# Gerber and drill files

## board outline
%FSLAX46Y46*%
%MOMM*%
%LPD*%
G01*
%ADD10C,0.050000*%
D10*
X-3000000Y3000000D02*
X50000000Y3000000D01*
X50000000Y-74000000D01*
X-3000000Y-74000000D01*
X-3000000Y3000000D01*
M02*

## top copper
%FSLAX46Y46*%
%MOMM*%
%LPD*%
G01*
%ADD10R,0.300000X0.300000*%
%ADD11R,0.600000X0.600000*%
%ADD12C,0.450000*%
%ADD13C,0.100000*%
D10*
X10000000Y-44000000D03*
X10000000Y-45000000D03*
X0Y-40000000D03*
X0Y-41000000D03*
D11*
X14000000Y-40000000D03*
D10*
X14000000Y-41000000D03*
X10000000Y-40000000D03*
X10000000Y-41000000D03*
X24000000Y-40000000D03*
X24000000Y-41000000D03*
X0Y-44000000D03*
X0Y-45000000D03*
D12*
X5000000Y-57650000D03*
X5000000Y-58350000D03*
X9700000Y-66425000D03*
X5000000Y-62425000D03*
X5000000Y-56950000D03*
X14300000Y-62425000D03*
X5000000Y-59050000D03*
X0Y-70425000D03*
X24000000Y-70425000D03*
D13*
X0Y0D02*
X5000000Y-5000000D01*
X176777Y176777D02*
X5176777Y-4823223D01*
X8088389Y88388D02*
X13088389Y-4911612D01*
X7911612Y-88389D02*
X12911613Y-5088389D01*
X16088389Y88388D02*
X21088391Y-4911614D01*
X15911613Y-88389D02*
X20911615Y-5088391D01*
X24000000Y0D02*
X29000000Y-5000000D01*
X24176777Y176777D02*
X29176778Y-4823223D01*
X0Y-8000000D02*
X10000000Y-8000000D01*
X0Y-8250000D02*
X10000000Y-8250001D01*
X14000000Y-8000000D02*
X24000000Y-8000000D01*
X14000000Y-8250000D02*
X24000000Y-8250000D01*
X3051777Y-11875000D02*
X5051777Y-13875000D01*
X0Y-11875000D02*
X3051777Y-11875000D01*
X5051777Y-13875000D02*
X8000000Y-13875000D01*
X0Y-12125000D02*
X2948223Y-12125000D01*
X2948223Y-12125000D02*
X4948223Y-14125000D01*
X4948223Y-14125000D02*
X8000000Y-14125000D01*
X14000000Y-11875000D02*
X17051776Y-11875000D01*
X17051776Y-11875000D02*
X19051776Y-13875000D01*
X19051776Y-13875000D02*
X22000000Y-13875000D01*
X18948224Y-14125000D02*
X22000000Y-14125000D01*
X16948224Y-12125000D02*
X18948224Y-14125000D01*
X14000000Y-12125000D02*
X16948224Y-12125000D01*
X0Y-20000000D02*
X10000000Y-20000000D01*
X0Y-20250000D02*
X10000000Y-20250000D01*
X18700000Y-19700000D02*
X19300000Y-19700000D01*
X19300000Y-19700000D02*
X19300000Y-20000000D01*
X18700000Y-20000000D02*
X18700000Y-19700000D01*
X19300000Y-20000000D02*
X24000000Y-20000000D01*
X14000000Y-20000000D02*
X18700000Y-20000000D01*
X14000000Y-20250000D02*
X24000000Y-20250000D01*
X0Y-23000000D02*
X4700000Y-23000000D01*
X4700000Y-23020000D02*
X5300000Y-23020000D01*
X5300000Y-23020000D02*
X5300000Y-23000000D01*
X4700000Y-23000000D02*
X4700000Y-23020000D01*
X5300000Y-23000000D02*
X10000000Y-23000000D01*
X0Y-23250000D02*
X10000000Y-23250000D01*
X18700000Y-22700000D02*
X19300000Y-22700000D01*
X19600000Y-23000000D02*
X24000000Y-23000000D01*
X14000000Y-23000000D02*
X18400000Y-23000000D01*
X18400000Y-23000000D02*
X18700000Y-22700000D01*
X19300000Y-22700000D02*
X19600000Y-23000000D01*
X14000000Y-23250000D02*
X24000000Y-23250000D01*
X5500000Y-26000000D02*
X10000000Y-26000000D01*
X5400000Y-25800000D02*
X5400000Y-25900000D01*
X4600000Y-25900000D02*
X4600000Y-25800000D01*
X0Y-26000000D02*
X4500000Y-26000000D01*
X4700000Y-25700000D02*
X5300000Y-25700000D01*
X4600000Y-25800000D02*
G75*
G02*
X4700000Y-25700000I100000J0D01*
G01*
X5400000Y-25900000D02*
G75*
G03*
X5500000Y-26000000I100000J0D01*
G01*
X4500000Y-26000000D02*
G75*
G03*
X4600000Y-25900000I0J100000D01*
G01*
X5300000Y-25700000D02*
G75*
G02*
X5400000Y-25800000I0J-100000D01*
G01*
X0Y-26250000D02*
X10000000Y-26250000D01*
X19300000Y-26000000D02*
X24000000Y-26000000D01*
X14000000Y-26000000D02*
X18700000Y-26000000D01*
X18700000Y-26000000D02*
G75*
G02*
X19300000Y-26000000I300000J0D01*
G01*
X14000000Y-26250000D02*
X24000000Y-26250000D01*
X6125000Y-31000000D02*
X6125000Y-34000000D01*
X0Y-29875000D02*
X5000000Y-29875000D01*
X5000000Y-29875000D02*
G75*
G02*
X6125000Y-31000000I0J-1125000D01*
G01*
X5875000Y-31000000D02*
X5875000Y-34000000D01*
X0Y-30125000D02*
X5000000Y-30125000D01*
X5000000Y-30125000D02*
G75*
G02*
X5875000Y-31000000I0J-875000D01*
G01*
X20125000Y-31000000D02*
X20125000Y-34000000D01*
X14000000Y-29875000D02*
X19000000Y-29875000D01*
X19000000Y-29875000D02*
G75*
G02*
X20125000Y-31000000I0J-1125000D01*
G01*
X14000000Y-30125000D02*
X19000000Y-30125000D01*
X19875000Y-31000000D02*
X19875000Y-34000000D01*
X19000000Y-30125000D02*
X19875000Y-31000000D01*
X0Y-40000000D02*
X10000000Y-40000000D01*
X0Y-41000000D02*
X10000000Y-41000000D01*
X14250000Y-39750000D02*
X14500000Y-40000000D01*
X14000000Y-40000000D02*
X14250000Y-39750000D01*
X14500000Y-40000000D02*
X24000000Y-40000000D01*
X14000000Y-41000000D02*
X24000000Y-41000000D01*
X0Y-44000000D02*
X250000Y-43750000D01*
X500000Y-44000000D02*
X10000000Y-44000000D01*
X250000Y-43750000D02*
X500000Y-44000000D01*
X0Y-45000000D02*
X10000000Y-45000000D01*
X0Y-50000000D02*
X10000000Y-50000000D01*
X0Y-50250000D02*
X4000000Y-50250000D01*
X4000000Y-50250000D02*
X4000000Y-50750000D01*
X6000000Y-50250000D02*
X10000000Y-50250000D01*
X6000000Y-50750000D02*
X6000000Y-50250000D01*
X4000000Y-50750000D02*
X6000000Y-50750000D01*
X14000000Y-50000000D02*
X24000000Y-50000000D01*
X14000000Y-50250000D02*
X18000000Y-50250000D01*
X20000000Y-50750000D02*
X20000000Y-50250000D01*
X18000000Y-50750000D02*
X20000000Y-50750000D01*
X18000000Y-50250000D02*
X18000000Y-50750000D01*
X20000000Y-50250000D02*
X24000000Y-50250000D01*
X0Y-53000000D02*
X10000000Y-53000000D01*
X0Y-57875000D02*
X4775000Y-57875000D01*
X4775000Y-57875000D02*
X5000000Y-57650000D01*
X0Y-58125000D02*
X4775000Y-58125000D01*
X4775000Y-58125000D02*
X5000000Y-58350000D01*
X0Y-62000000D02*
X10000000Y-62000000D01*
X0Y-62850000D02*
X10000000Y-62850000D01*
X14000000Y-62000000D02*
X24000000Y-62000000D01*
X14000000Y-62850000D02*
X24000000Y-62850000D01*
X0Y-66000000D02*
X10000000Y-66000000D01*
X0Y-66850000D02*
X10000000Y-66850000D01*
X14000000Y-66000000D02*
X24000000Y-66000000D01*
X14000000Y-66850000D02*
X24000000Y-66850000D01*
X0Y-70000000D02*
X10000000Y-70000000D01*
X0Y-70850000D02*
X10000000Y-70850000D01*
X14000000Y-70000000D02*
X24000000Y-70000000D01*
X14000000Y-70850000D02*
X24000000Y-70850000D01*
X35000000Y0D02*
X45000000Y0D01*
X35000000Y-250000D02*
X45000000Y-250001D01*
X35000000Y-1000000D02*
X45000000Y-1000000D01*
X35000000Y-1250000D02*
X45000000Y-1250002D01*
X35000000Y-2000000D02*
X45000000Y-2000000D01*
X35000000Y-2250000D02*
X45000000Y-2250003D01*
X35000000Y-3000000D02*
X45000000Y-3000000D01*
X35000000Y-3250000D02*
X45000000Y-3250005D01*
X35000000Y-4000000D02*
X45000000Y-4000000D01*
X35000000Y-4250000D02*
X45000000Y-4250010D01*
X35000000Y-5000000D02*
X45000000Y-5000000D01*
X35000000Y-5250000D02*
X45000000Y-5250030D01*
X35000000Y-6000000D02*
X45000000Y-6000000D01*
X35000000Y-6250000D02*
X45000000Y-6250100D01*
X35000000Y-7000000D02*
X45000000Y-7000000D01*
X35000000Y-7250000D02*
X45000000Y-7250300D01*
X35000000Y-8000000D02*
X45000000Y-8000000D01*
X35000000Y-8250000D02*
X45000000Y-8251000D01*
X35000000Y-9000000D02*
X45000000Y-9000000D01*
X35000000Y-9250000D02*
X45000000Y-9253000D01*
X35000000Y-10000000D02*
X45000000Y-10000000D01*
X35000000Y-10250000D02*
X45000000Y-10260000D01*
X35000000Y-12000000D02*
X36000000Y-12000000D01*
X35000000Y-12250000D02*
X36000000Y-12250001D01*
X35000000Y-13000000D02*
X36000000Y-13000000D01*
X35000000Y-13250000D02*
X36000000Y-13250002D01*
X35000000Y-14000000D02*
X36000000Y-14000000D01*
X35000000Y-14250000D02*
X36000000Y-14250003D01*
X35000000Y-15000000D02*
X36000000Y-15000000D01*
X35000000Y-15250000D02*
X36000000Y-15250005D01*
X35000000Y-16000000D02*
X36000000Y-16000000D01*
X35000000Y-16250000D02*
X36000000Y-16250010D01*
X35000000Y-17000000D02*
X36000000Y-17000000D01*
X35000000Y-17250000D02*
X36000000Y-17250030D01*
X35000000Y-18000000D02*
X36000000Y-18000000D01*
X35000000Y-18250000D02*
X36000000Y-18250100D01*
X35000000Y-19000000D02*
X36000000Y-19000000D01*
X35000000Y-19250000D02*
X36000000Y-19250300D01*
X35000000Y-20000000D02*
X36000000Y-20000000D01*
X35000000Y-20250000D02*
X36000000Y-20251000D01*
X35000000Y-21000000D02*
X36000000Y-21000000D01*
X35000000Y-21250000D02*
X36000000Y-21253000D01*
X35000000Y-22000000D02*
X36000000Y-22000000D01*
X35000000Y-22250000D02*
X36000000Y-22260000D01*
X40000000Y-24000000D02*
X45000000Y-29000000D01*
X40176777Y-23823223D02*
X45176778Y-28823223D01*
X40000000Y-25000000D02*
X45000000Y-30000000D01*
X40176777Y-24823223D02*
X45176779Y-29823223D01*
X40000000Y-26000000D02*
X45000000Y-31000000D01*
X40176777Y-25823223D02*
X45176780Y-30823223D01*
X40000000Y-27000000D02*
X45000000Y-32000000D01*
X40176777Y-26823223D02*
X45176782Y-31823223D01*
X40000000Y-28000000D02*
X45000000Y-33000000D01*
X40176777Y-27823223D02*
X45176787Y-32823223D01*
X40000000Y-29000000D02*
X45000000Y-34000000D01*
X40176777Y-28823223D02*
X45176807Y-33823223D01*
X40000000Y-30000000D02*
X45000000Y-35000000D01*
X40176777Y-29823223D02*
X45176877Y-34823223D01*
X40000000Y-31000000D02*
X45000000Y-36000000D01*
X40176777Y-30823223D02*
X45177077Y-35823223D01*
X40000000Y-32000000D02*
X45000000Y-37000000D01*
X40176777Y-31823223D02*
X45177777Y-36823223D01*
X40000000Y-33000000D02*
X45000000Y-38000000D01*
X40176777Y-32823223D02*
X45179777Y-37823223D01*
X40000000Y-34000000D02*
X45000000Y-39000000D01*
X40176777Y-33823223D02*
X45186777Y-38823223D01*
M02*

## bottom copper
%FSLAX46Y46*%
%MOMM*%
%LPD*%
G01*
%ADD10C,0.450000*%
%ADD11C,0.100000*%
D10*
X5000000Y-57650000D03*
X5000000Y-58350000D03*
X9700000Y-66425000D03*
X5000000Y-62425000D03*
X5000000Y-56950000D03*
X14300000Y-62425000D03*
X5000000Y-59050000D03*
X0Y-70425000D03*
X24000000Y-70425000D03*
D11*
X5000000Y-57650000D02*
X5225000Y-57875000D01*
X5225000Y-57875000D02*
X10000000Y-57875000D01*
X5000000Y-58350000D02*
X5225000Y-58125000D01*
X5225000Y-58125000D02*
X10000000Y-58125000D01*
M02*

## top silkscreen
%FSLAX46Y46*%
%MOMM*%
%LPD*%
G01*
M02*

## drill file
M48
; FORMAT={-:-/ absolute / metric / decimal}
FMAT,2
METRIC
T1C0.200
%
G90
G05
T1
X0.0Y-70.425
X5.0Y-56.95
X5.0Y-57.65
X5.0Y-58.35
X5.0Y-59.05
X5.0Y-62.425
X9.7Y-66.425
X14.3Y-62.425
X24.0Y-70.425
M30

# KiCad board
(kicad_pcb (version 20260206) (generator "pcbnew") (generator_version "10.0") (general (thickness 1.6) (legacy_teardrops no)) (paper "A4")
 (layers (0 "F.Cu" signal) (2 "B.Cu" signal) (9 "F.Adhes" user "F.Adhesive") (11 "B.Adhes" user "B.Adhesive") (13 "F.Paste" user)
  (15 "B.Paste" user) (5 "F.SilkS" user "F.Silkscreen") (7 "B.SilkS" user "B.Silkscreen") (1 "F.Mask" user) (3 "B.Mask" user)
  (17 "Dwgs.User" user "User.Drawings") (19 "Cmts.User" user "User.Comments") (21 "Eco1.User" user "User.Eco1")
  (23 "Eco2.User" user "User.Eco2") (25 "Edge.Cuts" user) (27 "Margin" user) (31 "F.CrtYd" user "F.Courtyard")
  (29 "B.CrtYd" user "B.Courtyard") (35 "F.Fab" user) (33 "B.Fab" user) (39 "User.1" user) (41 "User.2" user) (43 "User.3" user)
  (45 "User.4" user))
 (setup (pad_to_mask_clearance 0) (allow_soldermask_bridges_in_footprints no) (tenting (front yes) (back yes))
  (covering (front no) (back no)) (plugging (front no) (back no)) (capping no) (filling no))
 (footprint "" (layer "F.Cu") (at 10 44)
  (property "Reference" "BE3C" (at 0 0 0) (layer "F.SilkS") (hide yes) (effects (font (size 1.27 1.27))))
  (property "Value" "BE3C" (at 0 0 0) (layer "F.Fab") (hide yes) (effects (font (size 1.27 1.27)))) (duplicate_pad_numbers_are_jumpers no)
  (pad "1" smd rect (at 0 0) (size 0.3 0.3) (layers "F.Cu" "F.Mask" "F.Paste") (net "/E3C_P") (thermal_bridge_angle 45))
  (pad "2" smd rect (at 0 1) (size 0.3 0.3) (layers "F.Cu" "F.Mask" "F.Paste") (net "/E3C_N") (thermal_bridge_angle 45)))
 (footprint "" (layer "F.Cu") (at 0 40)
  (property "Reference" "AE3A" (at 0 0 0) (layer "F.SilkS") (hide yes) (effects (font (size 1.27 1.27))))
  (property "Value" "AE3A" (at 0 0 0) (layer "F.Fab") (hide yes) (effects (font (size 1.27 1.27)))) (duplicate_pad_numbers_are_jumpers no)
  (pad "1" smd rect (at 0 0) (size 0.3 0.3) (layers "F.Cu" "F.Mask" "F.Paste") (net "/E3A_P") (die_length 1) (thermal_bridge_angle 45))
  (pad "2" smd rect (at 0 1) (size 0.3 0.3) (layers "F.Cu" "F.Mask" "F.Paste") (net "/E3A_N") (thermal_bridge_angle 45)))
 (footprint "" (layer "F.Cu") (at 14 40)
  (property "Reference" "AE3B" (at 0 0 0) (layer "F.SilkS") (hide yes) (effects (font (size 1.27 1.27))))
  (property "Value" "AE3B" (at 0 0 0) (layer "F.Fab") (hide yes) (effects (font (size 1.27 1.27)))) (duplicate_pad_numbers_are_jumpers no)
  (pad "1" smd rect (at 0 0) (size 0.6 0.6) (layers "F.Cu" "F.Mask" "F.Paste") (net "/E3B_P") (thermal_bridge_angle 45))
  (pad "2" smd rect (at 0 1) (size 0.3 0.3) (layers "F.Cu" "F.Mask" "F.Paste") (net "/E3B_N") (thermal_bridge_angle 45)))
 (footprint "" (layer "F.Cu") (at 10 40)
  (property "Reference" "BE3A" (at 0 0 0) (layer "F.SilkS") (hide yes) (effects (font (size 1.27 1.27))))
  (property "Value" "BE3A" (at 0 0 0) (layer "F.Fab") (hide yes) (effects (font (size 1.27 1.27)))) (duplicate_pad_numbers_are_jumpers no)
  (pad "1" smd rect (at 0 0) (size 0.3 0.3) (layers "F.Cu" "F.Mask" "F.Paste") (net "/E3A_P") (thermal_bridge_angle 45))
  (pad "2" smd rect (at 0 1) (size 0.3 0.3) (layers "F.Cu" "F.Mask" "F.Paste") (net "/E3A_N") (thermal_bridge_angle 45)))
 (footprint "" (layer "F.Cu") (at 24 40)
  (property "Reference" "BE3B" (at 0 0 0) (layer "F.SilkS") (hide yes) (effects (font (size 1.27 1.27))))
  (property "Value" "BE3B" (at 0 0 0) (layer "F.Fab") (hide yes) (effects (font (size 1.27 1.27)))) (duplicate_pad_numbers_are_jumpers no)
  (pad "1" smd rect (at 0 0) (size 0.3 0.3) (layers "F.Cu" "F.Mask" "F.Paste") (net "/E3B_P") (thermal_bridge_angle 45))
  (pad "2" smd rect (at 0 1) (size 0.3 0.3) (layers "F.Cu" "F.Mask" "F.Paste") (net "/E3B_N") (thermal_bridge_angle 45)))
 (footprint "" (layer "F.Cu") (at 0 44)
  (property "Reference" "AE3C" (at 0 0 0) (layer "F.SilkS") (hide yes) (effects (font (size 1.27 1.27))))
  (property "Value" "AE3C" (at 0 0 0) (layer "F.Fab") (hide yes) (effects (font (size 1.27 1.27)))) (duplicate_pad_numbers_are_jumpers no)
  (pad "1" smd rect (at 0 0) (size 0.3 0.3) (layers "F.Cu" "F.Mask" "F.Paste") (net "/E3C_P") (thermal_bridge_angle 45))
  (pad "2" smd rect (at 0 1) (size 0.3 0.3) (layers "F.Cu" "F.Mask" "F.Paste") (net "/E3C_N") (thermal_bridge_angle 45)))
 (gr_rect (start -3 -3) (end 50 74) (stroke (width 0.05) (type default)) (fill no) (layer "Edge.Cuts"))
 (segment (start 0 0) (end 5 5) (width 0.1) (layer "F.Cu") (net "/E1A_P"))
 (segment (start 0.176777 -0.176777) (end 5.176777 4.823223) (width 0.1) (layer "F.Cu") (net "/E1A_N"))
 (segment (start 8.088389 -0.088388) (end 13.088389 4.911612) (width 0.1) (layer "F.Cu") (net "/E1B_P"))
 (segment (start 7.911612 0.088389) (end 12.911613 5.088389) (width 0.1) (layer "F.Cu") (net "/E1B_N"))
 (segment (start 16.088389 -0.088388) (end 21.088391 4.911614) (width 0.1) (layer "F.Cu") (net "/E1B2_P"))
 (segment (start 15.911613 0.088389) (end 20.911615 5.088391) (width 0.1) (layer "F.Cu") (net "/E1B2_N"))
 (segment (start 24 0) (end 29 5) (width 0.1) (layer "F.Cu") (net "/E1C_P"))
 (segment (start 24.176777 -0.176777) (end 29.176778 4.823223) (width 0.1) (layer "F.Cu") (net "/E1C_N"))
 (segment (start 0 8) (end 10 8) (width 0.1) (layer "F.Cu") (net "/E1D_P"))
 (segment (start 0 8.25) (end 10 8.250001) (width 0.1) (layer "F.Cu") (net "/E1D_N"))
 (segment (start 14 8) (end 24 8) (width 0.1) (layer "F.Cu") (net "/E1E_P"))
 (segment (start 14 8.25) (end 24 8.25) (width 0.1) (layer "F.Cu") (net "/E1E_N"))
 (segment (start 3.051777 11.875) (end 5.051777 13.875) (width 0.1) (layer "F.Cu") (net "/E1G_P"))
 (segment (start 0 11.875) (end 3.051777 11.875) (width 0.1) (layer "F.Cu") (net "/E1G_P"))
 (segment (start 5.051777 13.875) (end 8 13.875) (width 0.1) (layer "F.Cu") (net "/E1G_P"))
 (segment (start 0 12.125) (end 2.948223 12.125) (width 0.1) (layer "F.Cu") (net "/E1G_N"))
 (segment (start 2.948223 12.125) (end 4.948223 14.125) (width 0.1) (layer "F.Cu") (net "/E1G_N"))
 (segment (start 4.948223 14.125) (end 8 14.125) (width 0.1) (layer "F.Cu") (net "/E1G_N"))
 (segment (start 14 11.875) (end 17.051776 11.875) (width 0.1) (layer "F.Cu") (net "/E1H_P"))
 (segment (start 17.051776 11.875) (end 19.051776 13.875) (width 0.1) (layer "F.Cu") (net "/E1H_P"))
 (segment (start 19.051776 13.875) (end 22 13.875) (width 0.1) (layer "F.Cu") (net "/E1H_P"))
 (segment (start 18.948224 14.125) (end 22 14.125) (width 0.1) (layer "F.Cu") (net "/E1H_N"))
 (segment (start 16.948224 12.125) (end 18.948224 14.125) (width 0.1) (layer "F.Cu") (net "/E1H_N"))
 (segment (start 14 12.125) (end 16.948224 12.125) (width 0.1) (layer "F.Cu") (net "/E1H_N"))
 (segment (start 0 20) (end 10 20) (width 0.1) (layer "F.Cu") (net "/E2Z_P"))
 (segment (start 0 20.25) (end 10 20.25) (width 0.1) (layer "F.Cu") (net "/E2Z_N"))
 (segment (start 18.7 19.7) (end 19.3 19.7) (width 0.1) (layer "F.Cu") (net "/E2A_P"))
 (segment (start 19.3 19.7) (end 19.3 20) (width 0.1) (layer "F.Cu") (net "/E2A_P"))
 (segment (start 18.7 20) (end 18.7 19.7) (width 0.1) (layer "F.Cu") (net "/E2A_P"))
 (segment (start 19.3 20) (end 24 20) (width 0.1) (layer "F.Cu") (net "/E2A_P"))
 (segment (start 14 20) (end 18.7 20) (width 0.1) (layer "F.Cu") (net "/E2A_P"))
 (segment (start 14 20.25) (end 24 20.25) (width 0.1) (layer "F.Cu") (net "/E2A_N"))
 (segment (start 0 23) (end 4.7 23) (width 0.1) (layer "F.Cu") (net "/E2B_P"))
 (segment (start 4.7 23.02) (end 5.3 23.02) (width 0.1) (layer "F.Cu") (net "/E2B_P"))
 (segment (start 5.3 23.02) (end 5.3 23) (width 0.1) (layer "F.Cu") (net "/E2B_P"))
 (segment (start 4.7 23) (end 4.7 23.02) (width 0.1) (layer "F.Cu") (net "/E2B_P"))
 (segment (start 5.3 23) (end 10 23) (width 0.1) (layer "F.Cu") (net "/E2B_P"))
 (segment (start 0 23.25) (end 10 23.25) (width 0.1) (layer "F.Cu") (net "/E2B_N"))
 (segment (start 18.7 22.7) (end 19.3 22.7) (width 0.1) (layer "F.Cu") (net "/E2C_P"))
 (segment (start 19.6 23) (end 24 23) (width 0.1) (layer "F.Cu") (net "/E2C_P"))
 (segment (start 14 23) (end 18.4 23) (width 0.1) (layer "F.Cu") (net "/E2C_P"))
 (segment (start 18.4 23) (end 18.7 22.7) (width 0.1) (layer "F.Cu") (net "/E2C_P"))
 (segment (start 19.3 22.7) (end 19.6 23) (width 0.1) (layer "F.Cu") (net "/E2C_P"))
 (segment (start 14 23.25) (end 24 23.25) (width 0.1) (layer "F.Cu") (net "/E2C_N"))
 (segment (start 5.5 26) (end 10 26) (width 0.1) (layer "F.Cu") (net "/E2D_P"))
 (segment (start 5.4 25.8) (end 5.4 25.9) (width 0.1) (layer "F.Cu") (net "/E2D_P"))
 (segment (start 4.6 25.9) (end 4.6 25.8) (width 0.1) (layer "F.Cu") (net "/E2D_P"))
 (segment (start 0 26) (end 4.5 26) (width 0.1) (layer "F.Cu") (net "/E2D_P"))
 (segment (start 4.7 25.7) (end 5.3 25.7) (width 0.1) (layer "F.Cu") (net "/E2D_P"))
 (arc (start 4.6 25.8) (mid 4.629289 25.729289) (end 4.7 25.7) (width 0.1) (layer "F.Cu") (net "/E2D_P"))
 (arc (start 5.4 25.9) (mid 5.429289 25.970711) (end 5.5 26) (width 0.1) (layer "F.Cu") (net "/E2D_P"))
 (arc (start 4.5 26) (mid 4.570711 25.970711) (end 4.6 25.9) (width 0.1) (layer "F.Cu") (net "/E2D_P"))
 (arc (start 5.3 25.7) (mid 5.370711 25.729289) (end 5.4 25.8) (width 0.1) (layer "F.Cu") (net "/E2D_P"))
 (segment (start 0 26.25) (end 10 26.25) (width 0.1) (layer "F.Cu") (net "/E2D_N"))
 (segment (start 19.3 26) (end 24 26) (width 0.1) (layer "F.Cu") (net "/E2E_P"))
 (segment (start 14 26) (end 18.7 26) (width 0.1) (layer "F.Cu") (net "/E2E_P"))
 (arc (start 18.7 26) (mid 19 25.7) (end 19.3 26) (width 0.1) (layer "F.Cu") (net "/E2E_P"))
 (segment (start 14 26.25) (end 24 26.25) (width 0.1) (layer "F.Cu") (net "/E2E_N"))
 (segment (start 6.125 31) (end 6.125 34) (width 0.1) (layer "F.Cu") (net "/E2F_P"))
 (segment (start 0 29.875) (end 5 29.875) (width 0.1) (layer "F.Cu") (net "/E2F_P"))
 (arc (start 5 29.875) (mid 5.795495 30.204505) (end 6.125 31) (width 0.1) (layer "F.Cu") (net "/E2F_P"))
 (segment (start 5.875 31) (end 5.875 34) (width 0.1) (layer "F.Cu") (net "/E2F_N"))
 (segment (start 0 30.125) (end 5 30.125) (width 0.1) (layer "F.Cu") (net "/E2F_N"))
 (arc (start 5 30.125) (mid 5.618718 30.381282) (end 5.875 31) (width 0.1) (layer "F.Cu") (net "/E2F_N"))
 (segment (start 20.125 31) (end 20.125 34) (width 0.1) (layer "F.Cu") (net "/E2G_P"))
 (segment (start 14 29.875) (end 19 29.875) (width 0.1) (layer "F.Cu") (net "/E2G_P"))
 (arc (start 19 29.875) (mid 19.795495 30.204505) (end 20.125 31) (width 0.1) (layer "F.Cu") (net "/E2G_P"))
 (segment (start 14 30.125) (end 19 30.125) (width 0.1) (layer "F.Cu") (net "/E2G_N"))
 (segment (start 19.875 31) (end 19.875 34) (width 0.1) (layer "F.Cu") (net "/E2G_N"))
 (segment (start 19 30.125) (end 19.875 31) (width 0.1) (layer "F.Cu") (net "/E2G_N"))
 (segment (start 0 40) (end 10 40) (width 0.1) (layer "F.Cu") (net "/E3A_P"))
 (segment (start 0 41) (end 10 41) (width 0.1) (layer "F.Cu") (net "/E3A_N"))
 (segment (start 14.25 39.75) (end 14.5 40) (width 0.1) (layer "F.Cu") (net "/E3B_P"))
 (segment (start 14 40) (end 14.25 39.75) (width 0.1) (layer "F.Cu") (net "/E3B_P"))
 (segment (start 14.5 40) (end 24 40) (width 0.1) (layer "F.Cu") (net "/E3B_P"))
 (segment (start 14 41) (end 24 41) (width 0.1) (layer "F.Cu") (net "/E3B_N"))
 (segment (start 0 44) (end 0.25 43.75) (width 0.1) (layer "F.Cu") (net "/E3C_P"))
 (segment (start 0.5 44) (end 10 44) (width 0.1) (layer "F.Cu") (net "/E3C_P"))
 (segment (start 0.25 43.75) (end 0.5 44) (width 0.1) (layer "F.Cu") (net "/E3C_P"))
 (segment (start 0 45) (end 10 45) (width 0.1) (layer "F.Cu") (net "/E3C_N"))
 (segment (start 0 50) (end 10 50) (width 0.1) (layer "F.Cu") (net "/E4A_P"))
 (segment (start 0 50.25) (end 4 50.25) (width 0.1) (layer "F.Cu") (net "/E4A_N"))
 (segment (start 4 50.25) (end 4 50.75) (width 0.1) (layer "F.Cu") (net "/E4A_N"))
 (segment (start 6 50.25) (end 10 50.25) (width 0.1) (layer "F.Cu") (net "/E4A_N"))
 (segment (start 6 50.75) (end 6 50.25) (width 0.1) (layer "F.Cu") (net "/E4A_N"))
 (segment (start 4 50.75) (end 6 50.75) (width 0.1) (layer "F.Cu") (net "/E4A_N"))
 (segment (start 14 50) (end 24 50) (width 0.1) (layer "F.Cu") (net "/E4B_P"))
 (segment (start 14 50.25) (end 18 50.25) (width 0.1) (layer "F.Cu") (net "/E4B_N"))
 (segment (start 20 50.75) (end 20 50.25) (width 0.1) (layer "F.Cu") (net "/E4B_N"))
 (segment (start 18 50.75) (end 20 50.75) (width 0.1) (layer "F.Cu") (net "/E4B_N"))
 (segment (start 18 50.25) (end 18 50.75) (width 0.1) (layer "F.Cu") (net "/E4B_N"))
 (segment (start 20 50.25) (end 24 50.25) (width 0.1) (layer "F.Cu") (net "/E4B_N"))
 (segment (start 0 53) (end 10 53) (width 0.1) (layer "F.Cu") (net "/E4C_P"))
 (segment (start 0 57.875) (end 4.775 57.875) (width 0.1) (layer "F.Cu") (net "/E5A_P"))
 (segment (start 4.775 57.875) (end 5 57.65) (width 0.1) (layer "F.Cu") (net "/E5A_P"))
 (via (at 5 57.65) (size 0.45) (drill 0.2) (layers "F.Cu" "B.Cu") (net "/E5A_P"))
 (segment (start 5 57.65) (end 5.225 57.875) (width 0.1) (layer "B.Cu") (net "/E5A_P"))
 (segment (start 5.225 57.875) (end 10 57.875) (width 0.1) (layer "B.Cu") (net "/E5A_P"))
 (segment (start 0 58.125) (end 4.775 58.125) (width 0.1) (layer "F.Cu") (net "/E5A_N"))
 (segment (start 4.775 58.125) (end 5 58.35) (width 0.1) (layer "F.Cu") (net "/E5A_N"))
 (via (at 5 58.35) (size 0.45) (drill 0.2) (layers "F.Cu" "B.Cu") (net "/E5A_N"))
 (segment (start 5 58.35) (end 5.225 58.125) (width 0.1) (layer "B.Cu") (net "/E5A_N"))
 (segment (start 5.225 58.125) (end 10 58.125) (width 0.1) (layer "B.Cu") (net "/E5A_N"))
 (via (at 9.7 66.425) (size 0.45) (drill 0.2) (layers "F.Cu" "B.Cu") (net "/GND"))
 (via (at 5 62.425) (size 0.45) (drill 0.2) (layers "F.Cu" "B.Cu") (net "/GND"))
 (via (at 5 56.95) (size 0.45) (drill 0.2) (layers "F.Cu" "B.Cu") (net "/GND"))
 (via (at 14.3 62.425) (size 0.45) (drill 0.2) (layers "F.Cu" "B.Cu") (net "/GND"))
 (via (at 5 59.05) (size 0.45) (drill 0.2) (layers "F.Cu" "B.Cu") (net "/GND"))
 (via (at 0 70.425) (size 0.45) (drill 0.2) (layers "F.Cu" "B.Cu") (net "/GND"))
 (via (at 24 70.425) (size 0.45) (drill 0.2) (layers "F.Cu" "B.Cu") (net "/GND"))
 (segment (start 0 62) (end 10 62) (width 0.1) (layer "F.Cu") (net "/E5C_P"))
 (segment (start 0 62.85) (end 10 62.85) (width 0.1) (layer "F.Cu") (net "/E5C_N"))
 (segment (start 14 62) (end 24 62) (width 0.1) (layer "F.Cu") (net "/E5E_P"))
 (segment (start 14 62.85) (end 24 62.85) (width 0.1) (layer "F.Cu") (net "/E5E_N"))
 (segment (start 0 66) (end 10 66) (width 0.1) (layer "F.Cu") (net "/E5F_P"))
 (segment (start 0 66.85) (end 10 66.85) (width 0.1) (layer "F.Cu") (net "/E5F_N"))
 (segment (start 14 66) (end 24 66) (width 0.1) (layer "F.Cu") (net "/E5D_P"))
 (segment (start 14 66.85) (end 24 66.85) (width 0.1) (layer "F.Cu") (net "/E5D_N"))
 (segment (start 0 70) (end 10 70) (width 0.1) (layer "F.Cu") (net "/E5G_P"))
 (segment (start 0 70.85) (end 10 70.85) (width 0.1) (layer "F.Cu") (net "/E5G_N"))
 (segment (start 14 70) (end 24 70) (width 0.1) (layer "F.Cu") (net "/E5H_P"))
 (segment (start 14 70.85) (end 24 70.85) (width 0.1) (layer "F.Cu") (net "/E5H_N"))
 (segment (start 35 0) (end 45 0) (width 0.1) (layer "F.Cu") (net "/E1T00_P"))
 (segment (start 35 0.25) (end 45 0.250001) (width 0.1) (layer "F.Cu") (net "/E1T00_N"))
 (segment (start 35 1) (end 45 1) (width 0.1) (layer "F.Cu") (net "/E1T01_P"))
 (segment (start 35 1.25) (end 45 1.250002) (width 0.1) (layer "F.Cu") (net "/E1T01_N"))
 (segment (start 35 2) (end 45 2) (width 0.1) (layer "F.Cu") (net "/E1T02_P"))
 (segment (start 35 2.25) (end 45 2.250003) (width 0.1) (layer "F.Cu") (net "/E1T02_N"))
 (segment (start 35 3) (end 45 3) (width 0.1) (layer "F.Cu") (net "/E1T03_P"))
 (segment (start 35 3.25) (end 45 3.250005) (width 0.1) (layer "F.Cu") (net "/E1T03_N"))
 (segment (start 35 4) (end 45 4) (width 0.1) (layer "F.Cu") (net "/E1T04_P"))
 (segment (start 35 4.25) (end 45 4.25001) (width 0.1) (layer "F.Cu") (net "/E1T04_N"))
 (segment (start 35 5) (end 45 5) (width 0.1) (layer "F.Cu") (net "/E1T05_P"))
 (segment (start 35 5.25) (end 45 5.25003) (width 0.1) (layer "F.Cu") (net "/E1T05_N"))
 (segment (start 35 6) (end 45 6) (width 0.1) (layer "F.Cu") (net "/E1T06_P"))
 (segment (start 35 6.25) (end 45 6.2501) (width 0.1) (layer "F.Cu") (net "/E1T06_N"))
 (segment (start 35 7) (end 45 7) (width 0.1) (layer "F.Cu") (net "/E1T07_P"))
 (segment (start 35 7.25) (end 45 7.2503) (width 0.1) (layer "F.Cu") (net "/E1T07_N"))
 (segment (start 35 8) (end 45 8) (width 0.1) (layer "F.Cu") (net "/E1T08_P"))
 (segment (start 35 8.25) (end 45 8.251) (width 0.1) (layer "F.Cu") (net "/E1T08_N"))
 (segment (start 35 9) (end 45 9) (width 0.1) (layer "F.Cu") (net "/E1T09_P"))
 (segment (start 35 9.25) (end 45 9.253) (width 0.1) (layer "F.Cu") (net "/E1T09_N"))
 (segment (start 35 10) (end 45 10) (width 0.1) (layer "F.Cu") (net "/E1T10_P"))
 (segment (start 35 10.25) (end 45 10.26) (width 0.1) (layer "F.Cu") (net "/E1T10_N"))
 (segment (start 35 12) (end 36 12) (width 0.1) (layer "F.Cu") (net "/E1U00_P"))
 (segment (start 35 12.25) (end 36 12.250001) (width 0.1) (layer "F.Cu") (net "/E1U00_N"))
 (segment (start 35 13) (end 36 13) (width 0.1) (layer "F.Cu") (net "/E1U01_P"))
 (segment (start 35 13.25) (end 36 13.250002) (width 0.1) (layer "F.Cu") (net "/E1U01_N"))
 (segment (start 35 14) (end 36 14) (width 0.1) (layer "F.Cu") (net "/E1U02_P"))
 (segment (start 35 14.25) (end 36 14.250003) (width 0.1) (layer "F.Cu") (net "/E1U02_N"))
 (segment (start 35 15) (end 36 15) (width 0.1) (layer "F.Cu") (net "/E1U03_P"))
 (segment (start 35 15.25) (end 36 15.250005) (width 0.1) (layer "F.Cu") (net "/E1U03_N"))
 (segment (start 35 16) (end 36 16) (width 0.1) (layer "F.Cu") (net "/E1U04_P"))
 (segment (start 35 16.25) (end 36 16.25001) (width 0.1) (layer "F.Cu") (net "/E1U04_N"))
 (segment (start 35 17) (end 36 17) (width 0.1) (layer "F.Cu") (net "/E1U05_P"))
 (segment (start 35 17.25) (end 36 17.25003) (width 0.1) (layer "F.Cu") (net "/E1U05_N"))
 (segment (start 35 18) (end 36 18) (width 0.1) (layer "F.Cu") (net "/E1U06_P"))
 (segment (start 35 18.25) (end 36 18.2501) (width 0.1) (layer "F.Cu") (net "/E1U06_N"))
 (segment (start 35 19) (end 36 19) (width 0.1) (layer "F.Cu") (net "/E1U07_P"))
 (segment (start 35 19.25) (end 36 19.2503) (width 0.1) (layer "F.Cu") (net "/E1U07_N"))
 (segment (start 35 20) (end 36 20) (width 0.1) (layer "F.Cu") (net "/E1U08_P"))
 (segment (start 35 20.25) (end 36 20.251) (width 0.1) (layer "F.Cu") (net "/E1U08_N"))
 (segment (start 35 21) (end 36 21) (width 0.1) (layer "F.Cu") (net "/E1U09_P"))
 (segment (start 35 21.25) (end 36 21.253) (width 0.1) (layer "F.Cu") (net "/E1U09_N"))
 (segment (start 35 22) (end 36 22) (width 0.1) (layer "F.Cu") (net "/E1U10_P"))
 (segment (start 35 22.25) (end 36 22.26) (width 0.1) (layer "F.Cu") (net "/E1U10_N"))
 (segment (start 40 24) (end 45 29) (width 0.1) (layer "F.Cu") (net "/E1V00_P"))
 (segment (start 40.176777 23.823223) (end 45.176778 28.823223) (width 0.1) (layer "F.Cu") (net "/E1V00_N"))
 (segment (start 40 25) (end 45 30) (width 0.1) (layer "F.Cu") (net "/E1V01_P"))
 (segment (start 40.176777 24.823223) (end 45.176779 29.823223) (width 0.1) (layer "F.Cu") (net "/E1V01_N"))
 (segment (start 40 26) (end 45 31) (width 0.1) (layer "F.Cu") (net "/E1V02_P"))
 (segment (start 40.176777 25.823223) (end 45.17678 30.823223) (width 0.1) (layer "F.Cu") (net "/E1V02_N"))
 (segment (start 40 27) (end 45 32) (width 0.1) (layer "F.Cu") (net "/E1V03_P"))
 (segment (start 40.176777 26.823223) (end 45.176782 31.823223) (width 0.1) (layer "F.Cu") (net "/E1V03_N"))
 (segment (start 40 28) (end 45 33) (width 0.1) (layer "F.Cu") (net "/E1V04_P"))
 (segment (start 40.176777 27.823223) (end 45.176787 32.823223) (width 0.1) (layer "F.Cu") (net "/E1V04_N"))
 (segment (start 40 29) (end 45 34) (width 0.1) (layer "F.Cu") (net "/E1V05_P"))
 (segment (start 40.176777 28.823223) (end 45.176807 33.823223) (width 0.1) (layer "F.Cu") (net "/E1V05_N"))
 (segment (start 40 30) (end 45 35) (width 0.1) (layer "F.Cu") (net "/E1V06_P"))
 (segment (start 40.176777 29.823223) (end 45.176877 34.823223) (width 0.1) (layer "F.Cu") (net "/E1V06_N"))
 (segment (start 40 31) (end 45 36) (width 0.1) (layer "F.Cu") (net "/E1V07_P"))
 (segment (start 40.176777 30.823223) (end 45.177077 35.823223) (width 0.1) (layer "F.Cu") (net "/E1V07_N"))
 (segment (start 40 32) (end 45 37) (width 0.1) (layer "F.Cu") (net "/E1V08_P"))
 (segment (start 40.176777 31.823223) (end 45.177777 36.823223) (width 0.1) (layer "F.Cu") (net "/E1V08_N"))
 (segment (start 40 33) (end 45 38) (width 0.1) (layer "F.Cu") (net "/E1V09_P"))
 (segment (start 40.176777 32.823223) (end 45.179777 37.823223) (width 0.1) (layer "F.Cu") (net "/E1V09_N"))
 (segment (start 40 34) (end 45 39) (width 0.1) (layer "F.Cu") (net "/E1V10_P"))
 (segment (start 40.176777 33.823223) (end 45.186777 38.823223) (width 0.1) (layer "F.Cu") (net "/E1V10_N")))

